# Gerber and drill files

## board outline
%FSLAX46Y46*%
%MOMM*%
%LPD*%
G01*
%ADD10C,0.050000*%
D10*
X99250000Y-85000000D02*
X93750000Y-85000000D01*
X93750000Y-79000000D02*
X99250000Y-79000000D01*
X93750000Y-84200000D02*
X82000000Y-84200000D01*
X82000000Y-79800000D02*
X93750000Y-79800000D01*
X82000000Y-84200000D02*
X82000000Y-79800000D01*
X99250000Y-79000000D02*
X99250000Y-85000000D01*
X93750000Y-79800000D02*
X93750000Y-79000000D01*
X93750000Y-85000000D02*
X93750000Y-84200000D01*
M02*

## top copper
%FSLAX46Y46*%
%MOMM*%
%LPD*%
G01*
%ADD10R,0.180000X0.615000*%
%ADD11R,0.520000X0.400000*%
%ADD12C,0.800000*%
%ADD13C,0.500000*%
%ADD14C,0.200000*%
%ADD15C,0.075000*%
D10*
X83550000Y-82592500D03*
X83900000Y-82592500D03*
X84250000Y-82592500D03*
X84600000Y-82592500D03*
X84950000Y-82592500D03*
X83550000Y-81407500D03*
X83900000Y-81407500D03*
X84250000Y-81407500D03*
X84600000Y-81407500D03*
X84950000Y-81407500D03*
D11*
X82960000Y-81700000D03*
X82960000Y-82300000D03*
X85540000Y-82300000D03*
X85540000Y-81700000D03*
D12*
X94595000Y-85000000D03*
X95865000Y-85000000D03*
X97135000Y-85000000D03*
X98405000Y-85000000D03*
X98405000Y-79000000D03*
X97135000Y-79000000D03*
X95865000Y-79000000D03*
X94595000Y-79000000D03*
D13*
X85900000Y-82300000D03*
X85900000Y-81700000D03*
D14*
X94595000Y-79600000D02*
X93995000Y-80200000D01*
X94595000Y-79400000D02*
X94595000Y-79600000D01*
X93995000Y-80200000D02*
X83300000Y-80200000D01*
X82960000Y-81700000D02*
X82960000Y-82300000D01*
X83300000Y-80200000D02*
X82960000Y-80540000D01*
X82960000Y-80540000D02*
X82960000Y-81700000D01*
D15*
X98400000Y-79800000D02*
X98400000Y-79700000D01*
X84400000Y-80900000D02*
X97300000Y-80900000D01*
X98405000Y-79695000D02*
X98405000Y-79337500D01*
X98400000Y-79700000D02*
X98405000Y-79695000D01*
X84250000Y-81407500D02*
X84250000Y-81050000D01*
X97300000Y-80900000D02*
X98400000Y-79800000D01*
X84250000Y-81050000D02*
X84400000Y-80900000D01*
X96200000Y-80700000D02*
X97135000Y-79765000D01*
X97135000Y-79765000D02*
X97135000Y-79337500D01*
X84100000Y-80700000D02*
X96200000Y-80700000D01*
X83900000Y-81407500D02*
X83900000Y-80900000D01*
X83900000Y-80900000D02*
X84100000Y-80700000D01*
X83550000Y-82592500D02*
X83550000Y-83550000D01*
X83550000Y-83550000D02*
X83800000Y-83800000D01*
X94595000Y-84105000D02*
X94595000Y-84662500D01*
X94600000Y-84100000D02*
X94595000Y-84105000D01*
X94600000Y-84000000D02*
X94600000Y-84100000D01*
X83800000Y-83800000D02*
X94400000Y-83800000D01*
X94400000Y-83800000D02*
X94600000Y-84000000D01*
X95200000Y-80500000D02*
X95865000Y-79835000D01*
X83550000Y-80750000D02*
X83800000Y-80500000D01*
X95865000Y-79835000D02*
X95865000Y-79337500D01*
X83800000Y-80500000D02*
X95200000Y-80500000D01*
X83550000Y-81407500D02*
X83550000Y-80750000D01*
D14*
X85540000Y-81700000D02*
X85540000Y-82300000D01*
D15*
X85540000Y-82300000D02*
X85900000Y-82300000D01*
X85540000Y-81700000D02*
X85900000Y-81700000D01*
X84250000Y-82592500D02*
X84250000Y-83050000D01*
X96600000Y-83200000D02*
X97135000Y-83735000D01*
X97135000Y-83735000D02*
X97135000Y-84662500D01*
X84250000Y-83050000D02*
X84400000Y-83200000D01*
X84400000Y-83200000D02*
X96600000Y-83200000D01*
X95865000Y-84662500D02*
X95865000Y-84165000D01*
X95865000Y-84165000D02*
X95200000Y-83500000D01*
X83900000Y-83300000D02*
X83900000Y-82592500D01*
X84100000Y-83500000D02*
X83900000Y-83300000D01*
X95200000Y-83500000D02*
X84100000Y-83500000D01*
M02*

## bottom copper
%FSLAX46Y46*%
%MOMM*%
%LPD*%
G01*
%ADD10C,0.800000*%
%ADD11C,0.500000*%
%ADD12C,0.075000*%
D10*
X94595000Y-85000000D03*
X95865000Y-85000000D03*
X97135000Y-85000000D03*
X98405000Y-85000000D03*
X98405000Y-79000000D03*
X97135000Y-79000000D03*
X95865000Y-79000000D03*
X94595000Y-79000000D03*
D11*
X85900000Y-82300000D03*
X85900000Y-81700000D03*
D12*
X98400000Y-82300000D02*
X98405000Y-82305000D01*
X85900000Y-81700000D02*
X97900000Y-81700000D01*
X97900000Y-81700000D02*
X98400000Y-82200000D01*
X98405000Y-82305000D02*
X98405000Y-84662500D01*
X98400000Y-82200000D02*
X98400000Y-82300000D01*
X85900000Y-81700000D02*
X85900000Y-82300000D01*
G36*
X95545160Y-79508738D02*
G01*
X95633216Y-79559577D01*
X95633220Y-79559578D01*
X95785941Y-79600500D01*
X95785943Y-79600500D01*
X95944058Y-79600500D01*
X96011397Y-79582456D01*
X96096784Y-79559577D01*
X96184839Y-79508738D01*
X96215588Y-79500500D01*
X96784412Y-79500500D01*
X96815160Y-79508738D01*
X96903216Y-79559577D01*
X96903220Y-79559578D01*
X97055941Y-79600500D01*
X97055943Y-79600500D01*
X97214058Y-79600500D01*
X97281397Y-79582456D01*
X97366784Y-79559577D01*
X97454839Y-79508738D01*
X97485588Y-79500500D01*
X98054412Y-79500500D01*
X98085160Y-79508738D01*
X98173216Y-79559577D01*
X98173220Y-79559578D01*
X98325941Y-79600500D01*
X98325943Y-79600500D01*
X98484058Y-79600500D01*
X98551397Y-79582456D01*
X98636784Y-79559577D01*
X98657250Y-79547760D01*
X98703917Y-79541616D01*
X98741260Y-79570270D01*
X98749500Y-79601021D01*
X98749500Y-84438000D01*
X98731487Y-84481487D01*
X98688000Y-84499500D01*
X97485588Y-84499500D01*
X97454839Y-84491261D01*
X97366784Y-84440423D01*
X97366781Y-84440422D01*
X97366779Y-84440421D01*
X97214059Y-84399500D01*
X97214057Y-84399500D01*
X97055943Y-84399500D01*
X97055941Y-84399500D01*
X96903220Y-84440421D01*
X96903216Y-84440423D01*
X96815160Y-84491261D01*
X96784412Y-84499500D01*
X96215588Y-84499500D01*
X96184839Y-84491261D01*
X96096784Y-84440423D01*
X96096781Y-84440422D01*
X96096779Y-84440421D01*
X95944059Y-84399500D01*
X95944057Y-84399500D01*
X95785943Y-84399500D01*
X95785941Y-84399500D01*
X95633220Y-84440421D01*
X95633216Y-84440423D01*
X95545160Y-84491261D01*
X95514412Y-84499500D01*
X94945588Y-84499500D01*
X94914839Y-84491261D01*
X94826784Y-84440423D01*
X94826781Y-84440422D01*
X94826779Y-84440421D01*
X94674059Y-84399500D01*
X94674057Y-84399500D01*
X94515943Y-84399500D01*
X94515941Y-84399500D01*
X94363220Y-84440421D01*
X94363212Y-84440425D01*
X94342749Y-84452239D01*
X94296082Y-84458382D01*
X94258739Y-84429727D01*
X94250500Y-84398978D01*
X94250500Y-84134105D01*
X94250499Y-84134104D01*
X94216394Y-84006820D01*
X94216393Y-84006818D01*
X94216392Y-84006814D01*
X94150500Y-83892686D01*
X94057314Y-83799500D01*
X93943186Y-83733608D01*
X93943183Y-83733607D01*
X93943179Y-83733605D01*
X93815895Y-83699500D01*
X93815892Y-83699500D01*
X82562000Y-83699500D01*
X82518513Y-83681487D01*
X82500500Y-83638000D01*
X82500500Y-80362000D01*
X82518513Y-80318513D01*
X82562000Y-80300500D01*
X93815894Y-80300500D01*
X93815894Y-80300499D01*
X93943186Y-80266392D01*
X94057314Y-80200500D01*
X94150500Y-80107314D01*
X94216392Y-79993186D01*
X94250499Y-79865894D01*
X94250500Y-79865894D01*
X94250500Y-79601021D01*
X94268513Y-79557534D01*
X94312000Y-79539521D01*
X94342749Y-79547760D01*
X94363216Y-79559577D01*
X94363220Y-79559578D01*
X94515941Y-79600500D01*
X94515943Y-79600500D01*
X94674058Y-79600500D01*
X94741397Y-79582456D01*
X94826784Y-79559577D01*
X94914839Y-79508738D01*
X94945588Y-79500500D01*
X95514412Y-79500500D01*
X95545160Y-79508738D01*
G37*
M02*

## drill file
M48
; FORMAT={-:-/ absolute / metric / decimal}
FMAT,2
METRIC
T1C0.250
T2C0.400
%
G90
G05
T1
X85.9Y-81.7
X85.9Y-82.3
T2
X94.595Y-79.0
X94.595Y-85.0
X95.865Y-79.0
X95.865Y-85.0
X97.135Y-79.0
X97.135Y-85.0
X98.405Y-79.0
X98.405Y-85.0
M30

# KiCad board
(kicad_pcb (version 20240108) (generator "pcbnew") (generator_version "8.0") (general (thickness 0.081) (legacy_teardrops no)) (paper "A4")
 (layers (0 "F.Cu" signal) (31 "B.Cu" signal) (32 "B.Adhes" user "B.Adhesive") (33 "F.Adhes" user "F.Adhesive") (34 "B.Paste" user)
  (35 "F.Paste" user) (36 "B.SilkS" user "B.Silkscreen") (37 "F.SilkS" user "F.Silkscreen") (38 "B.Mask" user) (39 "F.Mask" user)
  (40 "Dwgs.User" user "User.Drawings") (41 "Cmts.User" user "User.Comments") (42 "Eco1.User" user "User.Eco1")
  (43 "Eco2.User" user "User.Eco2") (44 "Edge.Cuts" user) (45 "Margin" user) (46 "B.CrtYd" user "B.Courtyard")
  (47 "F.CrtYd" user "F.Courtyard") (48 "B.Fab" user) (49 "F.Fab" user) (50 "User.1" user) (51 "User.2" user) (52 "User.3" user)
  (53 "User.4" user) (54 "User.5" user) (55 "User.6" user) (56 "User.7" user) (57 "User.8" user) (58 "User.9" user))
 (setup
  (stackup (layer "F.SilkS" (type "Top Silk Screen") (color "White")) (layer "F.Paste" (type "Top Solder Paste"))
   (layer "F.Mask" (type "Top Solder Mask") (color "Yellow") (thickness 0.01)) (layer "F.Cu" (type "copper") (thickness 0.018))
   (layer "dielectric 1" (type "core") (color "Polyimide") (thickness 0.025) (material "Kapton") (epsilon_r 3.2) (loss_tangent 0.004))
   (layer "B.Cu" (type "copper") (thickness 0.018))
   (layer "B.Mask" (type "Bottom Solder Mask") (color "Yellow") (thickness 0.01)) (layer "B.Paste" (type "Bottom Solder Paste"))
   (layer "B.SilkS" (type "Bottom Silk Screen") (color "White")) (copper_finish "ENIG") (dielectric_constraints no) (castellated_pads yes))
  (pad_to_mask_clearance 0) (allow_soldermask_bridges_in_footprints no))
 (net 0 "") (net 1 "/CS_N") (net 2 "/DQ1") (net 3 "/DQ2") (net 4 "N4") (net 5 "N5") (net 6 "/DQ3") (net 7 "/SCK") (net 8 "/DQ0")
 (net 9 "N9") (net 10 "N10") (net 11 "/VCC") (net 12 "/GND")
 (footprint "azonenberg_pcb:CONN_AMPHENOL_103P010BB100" (layer "F.Cu") (at 84.25 82)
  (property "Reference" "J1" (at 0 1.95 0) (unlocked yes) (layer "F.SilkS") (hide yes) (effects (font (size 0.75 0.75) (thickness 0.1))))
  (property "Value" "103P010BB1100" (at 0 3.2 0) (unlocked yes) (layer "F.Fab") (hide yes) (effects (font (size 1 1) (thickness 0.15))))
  (pad "1" smd rect (at -0.7 0.5925) (size 0.18 0.615) (layers "F.Cu" "F.Paste" "F.Mask") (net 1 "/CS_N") (thermal_bridge_angle 45))
  (pad "2" smd rect (at -0.35 0.5925) (size 0.18 0.615) (layers "F.Cu" "F.Paste" "F.Mask") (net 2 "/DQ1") (thermal_bridge_angle 45))
  (pad "3" smd rect (at 0 0.5925) (size 0.18 0.615) (layers "F.Cu" "F.Paste" "F.Mask") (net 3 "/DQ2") (thermal_bridge_angle 45))
  (pad "4" smd rect (at 0.35 0.5925) (size 0.18 0.615) (layers "F.Cu" "F.Paste" "F.Mask") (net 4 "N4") (thermal_bridge_angle 45))
  (pad "5" smd rect (at 0.7 0.5925) (size 0.18 0.615) (layers "F.Cu" "F.Paste" "F.Mask") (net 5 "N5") (thermal_bridge_angle 45))
  (pad "6" smd rect (at -0.7 -0.5925) (size 0.18 0.615) (layers "F.Cu" "F.Paste" "F.Mask") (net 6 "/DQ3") (thermal_bridge_angle 45))
  (pad "7" smd rect (at -0.35 -0.5925) (size 0.18 0.615) (layers "F.Cu" "F.Paste" "F.Mask") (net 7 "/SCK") (thermal_bridge_angle 45))
  (pad "8" smd rect (at 0 -0.5925) (size 0.18 0.615) (layers "F.Cu" "F.Paste" "F.Mask") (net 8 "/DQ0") (thermal_bridge_angle 45))
  (pad "9" smd rect (at 0.35 -0.5925) (size 0.18 0.615) (layers "F.Cu" "F.Paste" "F.Mask") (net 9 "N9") (thermal_bridge_angle 45))
  (pad "10" smd rect (at 0.7 -0.5925) (size 0.18 0.615) (layers "F.Cu" "F.Paste" "F.Mask") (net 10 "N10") (thermal_bridge_angle 45))
  (pad "11" smd rect (at -1.29 -0.3) (size 0.52 0.4) (layers "F.Cu" "F.Paste" "F.Mask") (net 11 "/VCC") (thermal_bridge_angle 45))
  (pad "12" smd rect (at -1.29 0.3) (size 0.52 0.4) (layers "F.Cu" "F.Paste" "F.Mask") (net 11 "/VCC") (thermal_bridge_angle 45))
  (pad "13" smd rect (at 1.29 0.3) (size 0.52 0.4) (layers "F.Cu" "F.Paste" "F.Mask") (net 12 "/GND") (thermal_bridge_angle 45))
  (pad "14" smd rect (at 1.29 -0.3) (size 0.52 0.4) (layers "F.Cu" "F.Paste" "F.Mask") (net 12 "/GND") (thermal_bridge_angle 45)))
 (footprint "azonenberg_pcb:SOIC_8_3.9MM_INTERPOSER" (layer "F.Cu") (at 96.5 82)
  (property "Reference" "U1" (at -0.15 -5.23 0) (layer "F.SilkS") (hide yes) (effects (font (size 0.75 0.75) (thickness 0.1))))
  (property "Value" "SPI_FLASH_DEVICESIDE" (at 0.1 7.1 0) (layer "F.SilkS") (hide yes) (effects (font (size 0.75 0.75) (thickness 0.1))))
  (pad "1" thru_hole circle (at -1.905 3) (size 0.8 0.8) (drill 0.4) (layers "*.Cu" "*.Mask") (remove_unused_layers no) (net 1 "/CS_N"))
  (pad "2" thru_hole circle (at -0.635 3) (size 0.8 0.8) (drill 0.4) (layers "*.Cu" "*.Mask") (remove_unused_layers no) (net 2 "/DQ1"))
  (pad "3" thru_hole circle (at 0.635 3) (size 0.8 0.8) (drill 0.4) (layers "*.Cu" "*.Mask") (remove_unused_layers no) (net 3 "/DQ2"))
  (pad "4" thru_hole circle (at 1.905 3) (size 0.8 0.8) (drill 0.4) (layers "*.Cu" "*.Mask") (remove_unused_layers no) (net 12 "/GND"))
  (pad "5" thru_hole circle (at 1.905 -3) (size 0.8 0.8) (drill 0.4) (layers "*.Cu" "*.Mask") (remove_unused_layers no) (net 8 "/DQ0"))
  (pad "6" thru_hole circle (at 0.635 -3) (size 0.8 0.8) (drill 0.4) (layers "*.Cu" "*.Mask") (remove_unused_layers no) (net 7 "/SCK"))
  (pad "7" thru_hole circle (at -0.635 -3) (size 0.8 0.8) (drill 0.4) (layers "*.Cu" "*.Mask") (remove_unused_layers no) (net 6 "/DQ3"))
  (pad "8" thru_hole circle (at -1.905 -3) (size 0.8 0.8) (drill 0.4) (layers "*.Cu" "*.Mask") (remove_unused_layers no) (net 11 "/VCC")))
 (gr_line (start 99.25 85) (end 93.75 85) (stroke (width 0.05) (type default)) (layer "Edge.Cuts"))
 (gr_line (start 93.75 79) (end 99.25 79) (stroke (width 0.05) (type default)) (layer "Edge.Cuts"))
 (gr_line (start 93.75 84.2) (end 82 84.2) (stroke (width 0.05) (type default)) (layer "Edge.Cuts"))
 (gr_line (start 82 79.8) (end 93.75 79.8) (stroke (width 0.05) (type default)) (layer "Edge.Cuts"))
 (gr_line (start 82 84.2) (end 82 79.8) (stroke (width 0.05) (type default)) (layer "Edge.Cuts"))
 (gr_line (start 99.25 79) (end 99.25 85) (stroke (width 0.05) (type default)) (layer "Edge.Cuts"))
 (gr_line (start 93.75 79.8) (end 93.75 79) (stroke (width 0.05) (type default)) (layer "Edge.Cuts"))
 (gr_line (start 93.75 85) (end 93.75 84.2) (stroke (width 0.05) (type default)) (layer "Edge.Cuts"))
 (segment (start 94.595 79.6) (end 93.995 80.2) (width 0.2) (layer "F.Cu") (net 11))
 (segment (start 94.595 79.4) (end 94.595 79.6) (width 0.2) (layer "F.Cu") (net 11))
 (segment (start 93.995 80.2) (end 83.3 80.2) (width 0.2) (layer "F.Cu") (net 11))
 (segment (start 82.96 81.7) (end 82.96 82.3) (width 0.2) (layer "F.Cu") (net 11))
 (segment (start 83.3 80.2) (end 82.96 80.54) (width 0.2) (layer "F.Cu") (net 11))
 (segment (start 82.96 80.54) (end 82.96 81.7) (width 0.2) (layer "F.Cu") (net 11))
 (segment (start 98.4 79.8) (end 98.4 79.7) (width 0.075) (layer "F.Cu") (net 8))
 (segment (start 84.4 80.9) (end 97.3 80.9) (width 0.075) (layer "F.Cu") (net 8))
 (segment (start 98.405 79.695) (end 98.405 79.3375) (width 0.075) (layer "F.Cu") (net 8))
 (segment (start 98.4 79.7) (end 98.405 79.695) (width 0.075) (layer "F.Cu") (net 8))
 (segment (start 84.25 81.4075) (end 84.25 81.05) (width 0.075) (layer "F.Cu") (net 8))
 (segment (start 97.3 80.9) (end 98.4 79.8) (width 0.075) (layer "F.Cu") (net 8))
 (segment (start 84.25 81.05) (end 84.4 80.9) (width 0.075) (layer "F.Cu") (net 8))
 (segment (start 96.2 80.7) (end 97.135 79.765) (width 0.075) (layer "F.Cu") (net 7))
 (segment (start 97.135 79.765) (end 97.135 79.3375) (width 0.075) (layer "F.Cu") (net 7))
 (segment (start 84.1 80.7) (end 96.2 80.7) (width 0.075) (layer "F.Cu") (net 7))
 (segment (start 83.9 81.4075) (end 83.9 80.9) (width 0.075) (layer "F.Cu") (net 7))
 (segment (start 83.9 80.9) (end 84.1 80.7) (width 0.075) (layer "F.Cu") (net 7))
 (segment (start 83.55 82.5925) (end 83.55 83.55) (width 0.075) (layer "F.Cu") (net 1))
 (segment (start 83.55 83.55) (end 83.8 83.8) (width 0.075) (layer "F.Cu") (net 1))
 (segment (start 94.595 84.105) (end 94.595 84.6625) (width 0.075) (layer "F.Cu") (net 1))
 (segment (start 94.6 84.1) (end 94.595 84.105) (width 0.075) (layer "F.Cu") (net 1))
 (segment (start 94.6 84) (end 94.6 84.1) (width 0.075) (layer "F.Cu") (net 1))
 (segment (start 83.8 83.8) (end 94.4 83.8) (width 0.075) (layer "F.Cu") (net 1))
 (segment (start 94.4 83.8) (end 94.6 84) (width 0.075) (layer "F.Cu") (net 1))
 (segment (start 95.2 80.5) (end 95.865 79.835) (width 0.075) (layer "F.Cu") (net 6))
 (segment (start 83.55 80.75) (end 83.8 80.5) (width 0.075) (layer "F.Cu") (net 6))
 (segment (start 95.865 79.835) (end 95.865 79.3375) (width 0.075) (layer "F.Cu") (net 6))
 (segment (start 83.8 80.5) (end 95.2 80.5) (width 0.075) (layer "F.Cu") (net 6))
 (segment (start 83.55 81.4075) (end 83.55 80.75) (width 0.075) (layer "F.Cu") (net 6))
 (segment (start 85.54 81.7) (end 85.54 82.3) (width 0.2) (layer "F.Cu") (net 12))
 (segment (start 85.54 82.3) (end 85.9 82.3) (width 0.075) (layer "F.Cu") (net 12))
 (segment (start 85.54 81.7) (end 85.9 81.7) (width 0.075) (layer "F.Cu") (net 12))
 (via (at 85.9 82.3) (size 0.5) (drill 0.25) (layers "F.Cu" "B.Cu") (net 12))
 (via (at 85.9 81.7) (size 0.5) (drill 0.25) (layers "F.Cu" "B.Cu") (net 12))
 (segment (start 98.4 82.3) (end 98.405 82.305) (width 0.075) (layer "B.Cu") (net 12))
 (segment (start 85.9 81.7) (end 97.9 81.7) (width 0.075) (layer "B.Cu") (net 12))
 (segment (start 97.9 81.7) (end 98.4 82.2) (width 0.075) (layer "B.Cu") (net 12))
 (segment (start 98.405 82.305) (end 98.405 84.6625) (width 0.075) (layer "B.Cu") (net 12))
 (segment (start 98.4 82.2) (end 98.4 82.3) (width 0.075) (layer "B.Cu") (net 12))
 (segment (start 85.9 81.7) (end 85.9 82.3) (width 0.075) (layer "B.Cu") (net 12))
 (segment (start 84.25 82.5925) (end 84.25 83.05) (width 0.075) (layer "F.Cu") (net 3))
 (segment (start 96.6 83.2) (end 97.135 83.735) (width 0.075) (layer "F.Cu") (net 3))
 (segment (start 97.135 83.735) (end 97.135 84.6625) (width 0.075) (layer "F.Cu") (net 3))
 (segment (start 84.25 83.05) (end 84.4 83.2) (width 0.075) (layer "F.Cu") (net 3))
 (segment (start 84.4 83.2) (end 96.6 83.2) (width 0.075) (layer "F.Cu") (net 3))
 (segment (start 95.865 84.6625) (end 95.865 84.165) (width 0.075) (layer "F.Cu") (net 2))
 (segment (start 95.865 84.165) (end 95.2 83.5) (width 0.075) (layer "F.Cu") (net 2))
 (segment (start 83.9 83.3) (end 83.9 82.5925) (width 0.075) (layer "F.Cu") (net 2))
 (segment (start 84.1 83.5) (end 83.9 83.3) (width 0.075) (layer "F.Cu") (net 2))
 (segment (start 95.2 83.5) (end 84.1 83.5) (width 0.075) (layer "F.Cu") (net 2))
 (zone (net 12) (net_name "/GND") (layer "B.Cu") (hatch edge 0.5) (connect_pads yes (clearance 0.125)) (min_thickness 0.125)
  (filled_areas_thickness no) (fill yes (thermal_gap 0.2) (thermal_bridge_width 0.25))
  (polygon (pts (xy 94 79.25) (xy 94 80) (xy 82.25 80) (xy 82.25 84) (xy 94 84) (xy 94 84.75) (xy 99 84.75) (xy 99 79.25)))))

